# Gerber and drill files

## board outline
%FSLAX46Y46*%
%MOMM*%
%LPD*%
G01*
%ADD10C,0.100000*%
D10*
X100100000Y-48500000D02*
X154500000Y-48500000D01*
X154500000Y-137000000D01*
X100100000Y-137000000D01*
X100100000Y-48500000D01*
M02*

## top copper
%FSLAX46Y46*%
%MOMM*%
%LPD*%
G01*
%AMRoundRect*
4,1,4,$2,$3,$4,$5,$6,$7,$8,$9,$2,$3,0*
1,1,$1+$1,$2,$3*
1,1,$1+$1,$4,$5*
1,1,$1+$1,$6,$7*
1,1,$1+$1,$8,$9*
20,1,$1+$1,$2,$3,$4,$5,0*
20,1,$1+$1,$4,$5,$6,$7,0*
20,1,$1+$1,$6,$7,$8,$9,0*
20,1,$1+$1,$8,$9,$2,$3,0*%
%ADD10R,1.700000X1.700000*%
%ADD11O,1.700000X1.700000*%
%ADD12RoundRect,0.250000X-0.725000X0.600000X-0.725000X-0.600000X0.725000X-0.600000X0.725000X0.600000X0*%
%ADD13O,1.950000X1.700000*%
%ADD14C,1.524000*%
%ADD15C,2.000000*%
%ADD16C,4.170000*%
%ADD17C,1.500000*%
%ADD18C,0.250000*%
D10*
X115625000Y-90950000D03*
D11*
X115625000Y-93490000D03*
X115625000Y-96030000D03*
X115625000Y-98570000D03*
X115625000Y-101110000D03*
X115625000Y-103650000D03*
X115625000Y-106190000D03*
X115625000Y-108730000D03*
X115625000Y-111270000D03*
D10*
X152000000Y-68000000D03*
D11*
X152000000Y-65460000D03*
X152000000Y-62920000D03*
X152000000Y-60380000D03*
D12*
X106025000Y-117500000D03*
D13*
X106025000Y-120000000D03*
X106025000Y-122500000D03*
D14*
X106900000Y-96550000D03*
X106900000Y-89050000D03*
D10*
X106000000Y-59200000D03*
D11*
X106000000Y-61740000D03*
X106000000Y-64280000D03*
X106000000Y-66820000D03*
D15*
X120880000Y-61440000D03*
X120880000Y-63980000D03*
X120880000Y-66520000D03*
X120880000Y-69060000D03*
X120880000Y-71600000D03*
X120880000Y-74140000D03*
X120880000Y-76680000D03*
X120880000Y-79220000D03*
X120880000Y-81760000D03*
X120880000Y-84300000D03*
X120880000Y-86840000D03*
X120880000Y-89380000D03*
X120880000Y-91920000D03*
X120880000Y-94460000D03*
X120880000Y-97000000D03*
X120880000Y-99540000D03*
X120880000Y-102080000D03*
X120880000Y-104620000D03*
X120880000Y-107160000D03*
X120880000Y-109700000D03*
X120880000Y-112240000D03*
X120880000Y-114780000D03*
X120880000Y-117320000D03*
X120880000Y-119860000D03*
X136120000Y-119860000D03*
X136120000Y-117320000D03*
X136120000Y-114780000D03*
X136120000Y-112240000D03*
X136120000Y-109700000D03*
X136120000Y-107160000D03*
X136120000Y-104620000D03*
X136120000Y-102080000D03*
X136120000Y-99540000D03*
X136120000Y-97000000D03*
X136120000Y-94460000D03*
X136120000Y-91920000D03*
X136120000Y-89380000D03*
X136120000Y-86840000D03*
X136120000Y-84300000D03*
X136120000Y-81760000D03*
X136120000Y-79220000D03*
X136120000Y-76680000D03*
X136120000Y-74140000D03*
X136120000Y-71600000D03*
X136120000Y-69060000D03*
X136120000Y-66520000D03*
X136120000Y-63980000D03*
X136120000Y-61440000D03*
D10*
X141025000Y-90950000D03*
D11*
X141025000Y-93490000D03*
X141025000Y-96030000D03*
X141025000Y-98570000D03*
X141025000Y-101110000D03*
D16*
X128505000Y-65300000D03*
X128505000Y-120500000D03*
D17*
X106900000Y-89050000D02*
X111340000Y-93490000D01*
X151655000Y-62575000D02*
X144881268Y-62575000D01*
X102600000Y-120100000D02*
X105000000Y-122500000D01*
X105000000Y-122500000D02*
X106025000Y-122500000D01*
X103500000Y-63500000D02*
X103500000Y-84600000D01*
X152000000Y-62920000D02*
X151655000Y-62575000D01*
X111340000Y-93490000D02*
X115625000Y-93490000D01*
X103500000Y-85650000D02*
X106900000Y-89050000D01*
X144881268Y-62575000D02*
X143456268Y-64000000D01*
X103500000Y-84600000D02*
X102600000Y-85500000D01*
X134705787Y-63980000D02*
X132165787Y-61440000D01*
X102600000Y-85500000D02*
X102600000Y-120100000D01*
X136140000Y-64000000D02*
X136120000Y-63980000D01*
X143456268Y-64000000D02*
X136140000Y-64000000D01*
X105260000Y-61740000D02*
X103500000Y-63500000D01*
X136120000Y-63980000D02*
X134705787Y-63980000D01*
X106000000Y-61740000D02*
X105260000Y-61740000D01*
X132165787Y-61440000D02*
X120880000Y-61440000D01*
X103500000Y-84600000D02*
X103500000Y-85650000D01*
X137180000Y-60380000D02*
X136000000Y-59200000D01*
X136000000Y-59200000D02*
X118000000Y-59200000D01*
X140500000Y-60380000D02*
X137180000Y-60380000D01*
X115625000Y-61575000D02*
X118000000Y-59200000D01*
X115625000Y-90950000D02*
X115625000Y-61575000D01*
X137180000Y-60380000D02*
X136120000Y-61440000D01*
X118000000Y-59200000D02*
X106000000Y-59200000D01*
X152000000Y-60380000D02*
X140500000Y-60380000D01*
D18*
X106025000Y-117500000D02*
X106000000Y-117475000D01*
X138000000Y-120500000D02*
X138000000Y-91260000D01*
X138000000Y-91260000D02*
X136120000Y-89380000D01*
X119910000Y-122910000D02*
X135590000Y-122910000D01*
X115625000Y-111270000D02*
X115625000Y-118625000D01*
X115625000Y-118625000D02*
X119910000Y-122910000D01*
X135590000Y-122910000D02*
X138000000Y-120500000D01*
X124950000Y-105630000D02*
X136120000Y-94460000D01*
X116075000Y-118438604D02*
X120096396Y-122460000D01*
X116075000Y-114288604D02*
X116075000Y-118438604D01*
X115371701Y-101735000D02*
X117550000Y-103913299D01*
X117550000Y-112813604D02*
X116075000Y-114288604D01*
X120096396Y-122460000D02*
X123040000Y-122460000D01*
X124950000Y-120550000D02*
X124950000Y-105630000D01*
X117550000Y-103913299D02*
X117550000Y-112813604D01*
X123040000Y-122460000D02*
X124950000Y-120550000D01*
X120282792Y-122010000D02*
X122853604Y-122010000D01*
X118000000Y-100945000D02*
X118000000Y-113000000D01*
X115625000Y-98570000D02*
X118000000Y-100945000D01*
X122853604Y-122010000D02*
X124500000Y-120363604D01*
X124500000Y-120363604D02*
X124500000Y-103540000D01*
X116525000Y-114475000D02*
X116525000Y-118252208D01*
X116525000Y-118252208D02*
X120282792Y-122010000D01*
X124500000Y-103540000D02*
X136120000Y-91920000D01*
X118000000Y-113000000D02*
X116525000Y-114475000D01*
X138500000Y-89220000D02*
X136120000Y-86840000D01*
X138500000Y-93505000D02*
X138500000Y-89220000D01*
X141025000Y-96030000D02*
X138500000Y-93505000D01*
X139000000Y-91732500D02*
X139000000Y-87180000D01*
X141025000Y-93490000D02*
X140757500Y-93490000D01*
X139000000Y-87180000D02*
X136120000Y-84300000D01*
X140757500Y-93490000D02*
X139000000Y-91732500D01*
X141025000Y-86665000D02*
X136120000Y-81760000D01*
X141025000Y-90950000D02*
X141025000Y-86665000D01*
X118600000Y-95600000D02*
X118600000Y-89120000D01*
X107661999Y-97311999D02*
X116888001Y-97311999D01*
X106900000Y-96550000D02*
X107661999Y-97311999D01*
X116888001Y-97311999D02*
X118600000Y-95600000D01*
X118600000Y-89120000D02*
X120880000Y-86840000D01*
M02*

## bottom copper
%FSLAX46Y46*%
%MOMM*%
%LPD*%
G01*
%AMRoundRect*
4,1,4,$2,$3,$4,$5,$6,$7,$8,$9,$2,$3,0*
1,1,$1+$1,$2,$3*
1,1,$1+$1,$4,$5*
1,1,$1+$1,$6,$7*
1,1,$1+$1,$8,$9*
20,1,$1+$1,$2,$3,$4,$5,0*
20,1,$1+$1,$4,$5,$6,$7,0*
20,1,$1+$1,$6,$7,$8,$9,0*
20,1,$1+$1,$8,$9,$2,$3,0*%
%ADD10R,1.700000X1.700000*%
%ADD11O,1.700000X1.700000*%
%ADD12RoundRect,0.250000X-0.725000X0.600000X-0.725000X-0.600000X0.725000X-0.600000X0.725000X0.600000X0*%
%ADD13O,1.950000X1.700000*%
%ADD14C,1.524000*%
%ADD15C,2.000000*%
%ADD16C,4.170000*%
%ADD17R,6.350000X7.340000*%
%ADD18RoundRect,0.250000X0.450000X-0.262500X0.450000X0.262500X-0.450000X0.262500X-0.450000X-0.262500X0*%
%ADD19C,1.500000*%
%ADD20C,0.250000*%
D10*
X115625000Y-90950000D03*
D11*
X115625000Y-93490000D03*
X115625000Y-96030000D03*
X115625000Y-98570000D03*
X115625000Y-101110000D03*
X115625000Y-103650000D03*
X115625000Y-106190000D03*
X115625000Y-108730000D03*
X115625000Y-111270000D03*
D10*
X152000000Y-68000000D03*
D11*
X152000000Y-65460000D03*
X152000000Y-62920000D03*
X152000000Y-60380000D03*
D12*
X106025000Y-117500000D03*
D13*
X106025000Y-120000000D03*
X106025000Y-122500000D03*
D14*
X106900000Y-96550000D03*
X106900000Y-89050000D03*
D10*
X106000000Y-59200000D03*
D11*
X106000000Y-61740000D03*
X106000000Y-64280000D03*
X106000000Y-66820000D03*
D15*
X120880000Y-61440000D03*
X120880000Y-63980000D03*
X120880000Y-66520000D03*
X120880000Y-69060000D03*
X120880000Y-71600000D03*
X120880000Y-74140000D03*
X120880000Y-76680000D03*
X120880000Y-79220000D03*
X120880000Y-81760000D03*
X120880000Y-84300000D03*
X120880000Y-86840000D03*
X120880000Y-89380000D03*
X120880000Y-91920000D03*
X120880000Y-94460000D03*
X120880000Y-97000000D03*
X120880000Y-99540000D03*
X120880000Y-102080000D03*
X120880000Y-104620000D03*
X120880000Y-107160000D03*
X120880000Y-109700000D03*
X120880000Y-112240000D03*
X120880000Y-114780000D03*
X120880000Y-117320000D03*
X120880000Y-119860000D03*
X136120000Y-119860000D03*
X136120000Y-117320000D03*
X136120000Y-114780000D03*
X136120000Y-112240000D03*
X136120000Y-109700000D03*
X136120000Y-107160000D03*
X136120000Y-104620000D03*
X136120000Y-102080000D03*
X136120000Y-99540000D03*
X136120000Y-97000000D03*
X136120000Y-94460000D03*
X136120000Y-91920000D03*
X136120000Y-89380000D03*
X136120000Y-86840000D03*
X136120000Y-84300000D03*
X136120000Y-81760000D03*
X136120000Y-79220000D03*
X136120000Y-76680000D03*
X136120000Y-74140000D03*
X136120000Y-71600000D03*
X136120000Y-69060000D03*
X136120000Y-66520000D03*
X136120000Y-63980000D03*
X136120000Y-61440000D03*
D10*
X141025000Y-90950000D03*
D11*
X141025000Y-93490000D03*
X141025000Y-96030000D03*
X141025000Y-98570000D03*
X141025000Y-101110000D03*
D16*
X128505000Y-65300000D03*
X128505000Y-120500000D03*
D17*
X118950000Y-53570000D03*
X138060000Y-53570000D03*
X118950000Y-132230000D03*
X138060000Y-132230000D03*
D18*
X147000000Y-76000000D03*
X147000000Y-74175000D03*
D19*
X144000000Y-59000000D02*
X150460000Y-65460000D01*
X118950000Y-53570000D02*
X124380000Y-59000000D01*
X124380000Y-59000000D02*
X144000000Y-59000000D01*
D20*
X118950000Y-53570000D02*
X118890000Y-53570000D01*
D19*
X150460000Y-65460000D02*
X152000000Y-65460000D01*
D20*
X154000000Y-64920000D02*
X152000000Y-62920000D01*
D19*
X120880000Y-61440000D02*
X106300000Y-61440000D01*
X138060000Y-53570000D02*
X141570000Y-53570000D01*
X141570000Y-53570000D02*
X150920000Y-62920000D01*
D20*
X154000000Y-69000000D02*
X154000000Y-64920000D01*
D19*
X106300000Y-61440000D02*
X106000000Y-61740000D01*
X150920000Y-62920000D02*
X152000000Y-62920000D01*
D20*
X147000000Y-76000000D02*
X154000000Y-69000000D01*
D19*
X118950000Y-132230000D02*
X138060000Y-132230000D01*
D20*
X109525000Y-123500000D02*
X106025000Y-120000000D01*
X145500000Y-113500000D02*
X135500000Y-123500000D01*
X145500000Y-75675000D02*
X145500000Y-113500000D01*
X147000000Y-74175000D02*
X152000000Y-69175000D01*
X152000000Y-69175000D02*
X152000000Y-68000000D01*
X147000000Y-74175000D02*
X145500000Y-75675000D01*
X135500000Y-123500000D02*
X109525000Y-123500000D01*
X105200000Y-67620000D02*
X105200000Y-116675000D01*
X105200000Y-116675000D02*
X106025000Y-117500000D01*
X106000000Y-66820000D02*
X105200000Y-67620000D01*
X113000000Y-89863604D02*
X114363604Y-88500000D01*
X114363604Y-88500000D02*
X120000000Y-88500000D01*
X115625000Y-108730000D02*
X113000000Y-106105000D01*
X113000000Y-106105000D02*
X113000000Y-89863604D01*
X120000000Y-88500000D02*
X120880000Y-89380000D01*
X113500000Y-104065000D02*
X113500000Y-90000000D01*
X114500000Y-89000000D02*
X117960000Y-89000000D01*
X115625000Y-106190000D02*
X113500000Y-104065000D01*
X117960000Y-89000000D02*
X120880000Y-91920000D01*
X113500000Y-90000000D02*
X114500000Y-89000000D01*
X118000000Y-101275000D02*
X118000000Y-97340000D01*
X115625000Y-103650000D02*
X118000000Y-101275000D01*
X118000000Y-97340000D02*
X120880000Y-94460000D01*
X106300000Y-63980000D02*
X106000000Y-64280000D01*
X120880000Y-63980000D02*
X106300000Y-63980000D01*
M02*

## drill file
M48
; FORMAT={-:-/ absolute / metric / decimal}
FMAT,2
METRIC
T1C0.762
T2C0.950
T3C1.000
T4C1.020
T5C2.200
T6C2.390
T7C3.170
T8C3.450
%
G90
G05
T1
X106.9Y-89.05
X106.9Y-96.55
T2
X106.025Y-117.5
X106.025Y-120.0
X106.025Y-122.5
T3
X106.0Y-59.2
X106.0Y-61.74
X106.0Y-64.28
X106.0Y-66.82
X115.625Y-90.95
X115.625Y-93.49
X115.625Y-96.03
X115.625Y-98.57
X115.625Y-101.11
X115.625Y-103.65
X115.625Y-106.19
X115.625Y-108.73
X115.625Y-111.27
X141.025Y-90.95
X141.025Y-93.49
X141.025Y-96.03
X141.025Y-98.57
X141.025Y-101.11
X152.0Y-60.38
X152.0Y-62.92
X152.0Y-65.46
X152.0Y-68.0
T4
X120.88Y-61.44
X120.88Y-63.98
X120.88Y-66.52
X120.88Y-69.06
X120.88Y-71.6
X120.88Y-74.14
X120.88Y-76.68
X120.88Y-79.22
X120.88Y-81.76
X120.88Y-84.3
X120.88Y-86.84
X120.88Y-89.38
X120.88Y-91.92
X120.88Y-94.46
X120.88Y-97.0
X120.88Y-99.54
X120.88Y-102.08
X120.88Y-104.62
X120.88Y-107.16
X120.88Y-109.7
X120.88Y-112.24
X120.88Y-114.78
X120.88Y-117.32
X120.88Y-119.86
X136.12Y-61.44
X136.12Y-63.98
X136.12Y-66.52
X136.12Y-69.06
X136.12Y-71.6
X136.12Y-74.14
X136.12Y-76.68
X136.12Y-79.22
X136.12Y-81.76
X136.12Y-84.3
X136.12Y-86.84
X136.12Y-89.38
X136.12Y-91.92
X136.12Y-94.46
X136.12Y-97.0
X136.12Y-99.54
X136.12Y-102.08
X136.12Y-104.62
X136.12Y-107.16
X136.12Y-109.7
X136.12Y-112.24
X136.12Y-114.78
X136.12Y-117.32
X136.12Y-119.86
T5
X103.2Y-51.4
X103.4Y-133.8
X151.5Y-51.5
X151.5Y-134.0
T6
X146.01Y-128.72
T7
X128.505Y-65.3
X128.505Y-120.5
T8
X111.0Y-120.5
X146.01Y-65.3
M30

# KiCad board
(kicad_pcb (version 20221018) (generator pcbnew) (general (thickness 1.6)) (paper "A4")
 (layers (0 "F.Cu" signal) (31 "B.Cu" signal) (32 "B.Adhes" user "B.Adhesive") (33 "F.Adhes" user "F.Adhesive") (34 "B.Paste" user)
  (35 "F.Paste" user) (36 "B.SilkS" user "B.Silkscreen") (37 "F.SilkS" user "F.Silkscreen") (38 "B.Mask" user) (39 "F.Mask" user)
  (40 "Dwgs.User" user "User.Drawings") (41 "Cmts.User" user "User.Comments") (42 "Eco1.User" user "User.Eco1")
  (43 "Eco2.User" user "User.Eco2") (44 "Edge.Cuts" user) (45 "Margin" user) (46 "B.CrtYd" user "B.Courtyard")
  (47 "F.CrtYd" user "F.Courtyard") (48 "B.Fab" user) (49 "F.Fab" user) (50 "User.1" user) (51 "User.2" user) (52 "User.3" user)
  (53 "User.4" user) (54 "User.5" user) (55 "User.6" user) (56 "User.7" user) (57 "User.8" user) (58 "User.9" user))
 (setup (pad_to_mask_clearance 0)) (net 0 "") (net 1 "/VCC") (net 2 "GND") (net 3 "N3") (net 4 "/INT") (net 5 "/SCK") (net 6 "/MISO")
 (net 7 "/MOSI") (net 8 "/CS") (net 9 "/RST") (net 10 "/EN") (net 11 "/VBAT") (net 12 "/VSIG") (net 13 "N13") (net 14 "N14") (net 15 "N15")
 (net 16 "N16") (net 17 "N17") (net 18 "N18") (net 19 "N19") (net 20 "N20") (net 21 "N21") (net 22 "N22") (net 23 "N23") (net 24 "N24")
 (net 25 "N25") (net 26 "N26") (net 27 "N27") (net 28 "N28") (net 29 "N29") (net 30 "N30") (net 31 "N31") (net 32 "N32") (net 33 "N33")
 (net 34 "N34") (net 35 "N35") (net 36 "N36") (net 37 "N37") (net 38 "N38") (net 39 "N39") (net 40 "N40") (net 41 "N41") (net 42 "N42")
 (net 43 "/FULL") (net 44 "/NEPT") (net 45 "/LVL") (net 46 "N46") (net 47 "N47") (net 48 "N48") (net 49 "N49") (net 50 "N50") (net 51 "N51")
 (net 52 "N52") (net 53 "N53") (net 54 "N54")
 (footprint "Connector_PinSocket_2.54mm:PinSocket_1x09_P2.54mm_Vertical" (layer "F.Cu") (at 115.625 90.95)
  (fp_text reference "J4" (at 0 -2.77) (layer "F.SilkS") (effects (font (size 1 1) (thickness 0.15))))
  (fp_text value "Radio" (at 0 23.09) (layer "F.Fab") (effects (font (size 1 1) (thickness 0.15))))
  (pad "1" thru_hole rect (at 0 0) (size 1.7 1.7) (drill 1) (layers "*.Cu" "*.Mask") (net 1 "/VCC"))
  (pad "2" thru_hole oval (at 0 2.54) (size 1.7 1.7) (drill 1) (layers "*.Cu" "*.Mask") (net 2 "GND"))
  (pad "3" thru_hole oval (at 0 5.08) (size 1.7 1.7) (drill 1) (layers "*.Cu" "*.Mask") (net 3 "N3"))
  (pad "4" thru_hole oval (at 0 7.62) (size 1.7 1.7) (drill 1) (layers "*.Cu" "*.Mask") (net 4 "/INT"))
  (pad "5" thru_hole oval (at 0 10.16) (size 1.7 1.7) (drill 1) (layers "*.Cu" "*.Mask") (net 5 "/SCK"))
  (pad "6" thru_hole oval (at 0 12.7) (size 1.7 1.7) (drill 1) (layers "*.Cu" "*.Mask") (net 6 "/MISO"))
  (pad "7" thru_hole oval (at 0 15.24) (size 1.7 1.7) (drill 1) (layers "*.Cu" "*.Mask") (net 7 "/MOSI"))
  (pad "8" thru_hole oval (at 0 17.78) (size 1.7 1.7) (drill 1) (layers "*.Cu" "*.Mask") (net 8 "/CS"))
  (pad "9" thru_hole oval (at 0 20.32) (size 1.7 1.7) (drill 1) (layers "*.Cu" "*.Mask") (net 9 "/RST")))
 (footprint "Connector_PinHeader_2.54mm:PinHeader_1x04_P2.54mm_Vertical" (layer "F.Cu") (at 152 68 180)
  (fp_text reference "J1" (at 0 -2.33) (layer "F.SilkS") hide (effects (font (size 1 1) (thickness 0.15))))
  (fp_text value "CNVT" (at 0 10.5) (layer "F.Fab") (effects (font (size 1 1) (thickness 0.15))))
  (pad "1" thru_hole rect (at 0 0 180) (size 1.7 1.7) (drill 1) (layers "*.Cu" "*.Mask") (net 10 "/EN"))
  (pad "2" thru_hole oval (at 0 2.54 180) (size 1.7 1.7) (drill 1) (layers "*.Cu" "*.Mask") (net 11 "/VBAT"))
  (pad "3" thru_hole oval (at 0 5.08 180) (size 1.7 1.7) (drill 1) (layers "*.Cu" "*.Mask") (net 2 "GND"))
  (pad "4" thru_hole oval (at 0 7.62 180) (size 1.7 1.7) (drill 1) (layers "*.Cu" "*.Mask") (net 1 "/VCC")))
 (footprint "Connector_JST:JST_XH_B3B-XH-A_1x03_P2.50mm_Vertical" (layer "F.Cu") (at 106.025 117.5 -90)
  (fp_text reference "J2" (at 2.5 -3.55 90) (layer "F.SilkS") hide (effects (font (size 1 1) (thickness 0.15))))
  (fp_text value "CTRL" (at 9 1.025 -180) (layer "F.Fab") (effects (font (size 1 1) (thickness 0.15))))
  (pad "1" thru_hole roundrect (at 0 0 270) (size 1.7 1.95) (drill 0.95) (layers "*.Cu" "*.Mask") (roundrect_rratio 0.1470588235)
   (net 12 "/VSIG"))
  (pad "2" thru_hole oval (at 2.5 0 270) (size 1.7 1.95) (drill 0.95) (layers "*.Cu" "*.Mask") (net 10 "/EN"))
  (pad "3" thru_hole oval (at 5 0 270) (size 1.7 1.95) (drill 0.95) (layers "*.Cu" "*.Mask") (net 2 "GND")))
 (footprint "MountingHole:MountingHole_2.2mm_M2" (layer "F.Cu") (at 151.5 134)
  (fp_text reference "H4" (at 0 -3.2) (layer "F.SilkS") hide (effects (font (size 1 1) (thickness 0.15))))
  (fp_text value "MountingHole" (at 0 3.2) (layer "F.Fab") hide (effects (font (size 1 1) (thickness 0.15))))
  (pad "" np_thru_hole circle (at 0 0) (size 2.2 2.2) (drill 2.2) (layers "*.Cu" "*.Mask")))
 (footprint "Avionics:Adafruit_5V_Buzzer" (layer "F.Cu") (at 111.4 92.8 90)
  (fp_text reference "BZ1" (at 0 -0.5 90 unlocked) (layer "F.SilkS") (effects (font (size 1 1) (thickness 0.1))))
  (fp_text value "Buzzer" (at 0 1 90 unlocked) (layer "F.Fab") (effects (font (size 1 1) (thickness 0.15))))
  (pad "1" thru_hole circle (at -3.75 -4.5 90) (size 1.524 1.524) (drill 0.762) (layers "*.Cu" "*.Mask") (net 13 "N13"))
  (pad "2" thru_hole circle (at 3.75 -4.5 90) (size 1.524 1.524) (drill 0.762) (layers "*.Cu" "*.Mask") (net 2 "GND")))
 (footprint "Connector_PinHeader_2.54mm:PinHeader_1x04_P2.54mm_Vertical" (layer "F.Cu") (at 106 59.2)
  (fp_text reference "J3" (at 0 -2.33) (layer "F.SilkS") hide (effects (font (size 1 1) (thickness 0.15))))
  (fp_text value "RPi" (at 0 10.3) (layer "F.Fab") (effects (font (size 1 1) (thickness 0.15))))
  (pad "1" thru_hole rect (at 0 0) (size 1.7 1.7) (drill 1) (layers "*.Cu" "*.Mask") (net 1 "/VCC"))
  (pad "2" thru_hole oval (at 0 2.54) (size 1.7 1.7) (drill 1) (layers "*.Cu" "*.Mask") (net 2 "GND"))
  (pad "3" thru_hole oval (at 0 5.08) (size 1.7 1.7) (drill 1) (layers "*.Cu" "*.Mask") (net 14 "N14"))
  (pad "4" thru_hole oval (at 0 7.62) (size 1.7 1.7) (drill 1) (layers "*.Cu" "*.Mask") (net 12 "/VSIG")))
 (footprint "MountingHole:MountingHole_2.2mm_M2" (layer "F.Cu") (at 151.5 51.5)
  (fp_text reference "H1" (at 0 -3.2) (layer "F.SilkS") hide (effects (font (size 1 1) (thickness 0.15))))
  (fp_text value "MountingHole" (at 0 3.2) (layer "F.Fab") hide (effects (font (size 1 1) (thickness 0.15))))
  (pad "" np_thru_hole circle (at 0 0) (size 2.2 2.2) (drill 2.2) (layers "*.Cu" "*.Mask")))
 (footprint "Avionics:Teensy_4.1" (layer "F.Cu") (at 128.5 90.65)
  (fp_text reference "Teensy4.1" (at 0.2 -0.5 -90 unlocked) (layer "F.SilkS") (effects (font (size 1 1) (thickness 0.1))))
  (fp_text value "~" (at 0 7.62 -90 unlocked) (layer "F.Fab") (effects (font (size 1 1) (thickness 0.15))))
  (pad "0" thru_hole circle (at -7.62 -29.21) (size 2 2) (drill 1.02) (layers "*.Cu" "*.Mask") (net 2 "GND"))
  (pad "1" thru_hole circle (at -7.62 -26.67) (size 2 2) (drill 1.02) (layers "*.Cu" "*.Mask") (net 14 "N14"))
  (pad "2" thru_hole circle (at -7.62 -24.13) (size 2 2) (drill 1.02) (layers "*.Cu" "*.Mask") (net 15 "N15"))
  (pad "3" thru_hole circle (at -7.62 -21.59) (size 2 2) (drill 1.02) (layers "*.Cu" "*.Mask") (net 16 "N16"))
  (pad "4" thru_hole circle (at -7.62 -19.05) (size 2 2) (drill 1.02) (layers "*.Cu" "*.Mask") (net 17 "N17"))
  (pad "5" thru_hole circle (at -7.62 -16.51) (size 2 2) (drill 1.02) (layers "*.Cu" "*.Mask") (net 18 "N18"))
  (pad "6" thru_hole circle (at -7.62 -13.97) (size 2 2) (drill 1.02) (layers "*.Cu" "*.Mask") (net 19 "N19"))
  (pad "7" thru_hole circle (at -7.62 -11.43) (size 2 2) (drill 1.02) (layers "*.Cu" "*.Mask") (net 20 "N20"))
  (pad "8" thru_hole circle (at -7.62 -8.89) (size 2 2) (drill 1.02) (layers "*.Cu" "*.Mask") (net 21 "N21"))
  (pad "9" thru_hole circle (at -7.62 -6.35) (size 2 2) (drill 1.02) (layers "*.Cu" "*.Mask") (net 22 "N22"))
  (pad "10" thru_hole circle (at -7.62 -3.81) (size 2 2) (drill 1.02) (layers "*.Cu" "*.Mask") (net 13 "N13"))
  (pad "11" thru_hole circle (at -7.62 -1.27) (size 2 2) (drill 1.02) (layers "*.Cu" "*.Mask") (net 8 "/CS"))
  (pad "12" thru_hole circle (at -7.62 1.27) (size 2 2) (drill 1.02) (layers "*.Cu" "*.Mask") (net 7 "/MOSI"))
  (pad "13" thru_hole circle (at -7.62 3.81) (size 2 2) (drill 1.02) (layers "*.Cu" "*.Mask") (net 6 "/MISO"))
  (pad "14" thru_hole circle (at -7.62 6.35) (size 2 2) (drill 1.02) (layers "*.Cu" "*.Mask") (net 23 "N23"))
  (pad "15" thru_hole circle (at -7.62 8.89) (size 2 2) (drill 1.02) (layers "*.Cu" "*.Mask") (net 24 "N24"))
  (pad "16" thru_hole circle (at -7.62 11.43) (size 2 2) (drill 1.02) (layers "*.Cu" "*.Mask") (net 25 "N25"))
  (pad "17" thru_hole circle (at -7.62 13.97) (size 2 2) (drill 1.02) (layers "*.Cu" "*.Mask") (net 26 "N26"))
  (pad "18" thru_hole circle (at -7.62 16.51) (size 2 2) (drill 1.02) (layers "*.Cu" "*.Mask") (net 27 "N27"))
  (pad "19" thru_hole circle (at -7.62 19.05) (size 2 2) (drill 1.02) (layers "*.Cu" "*.Mask") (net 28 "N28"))
  (pad "20" thru_hole circle (at -7.62 21.59) (size 2 2) (drill 1.02) (layers "*.Cu" "*.Mask") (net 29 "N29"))
  (pad "21" thru_hole circle (at -7.62 24.13) (size 2 2) (drill 1.02) (layers "*.Cu" "*.Mask") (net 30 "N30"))
  (pad "22" thru_hole circle (at -7.62 26.67) (size 2 2) (drill 1.02) (layers "*.Cu" "*.Mask") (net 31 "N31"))
  (pad "23" thru_hole circle (at -7.62 29.21) (size 2 2) (drill 1.02) (layers "*.Cu" "*.Mask") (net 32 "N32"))
  (pad "24" thru_hole circle (at 7.62 29.21) (size 2 2) (drill 1.02) (layers "*.Cu" "*.Mask") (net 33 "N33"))
  (pad "25" thru_hole circle (at 7.62 26.67) (size 2 2) (drill 1.02) (layers "*.Cu" "*.Mask") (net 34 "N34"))
  (pad "26" thru_hole circle (at 7.62 24.13) (size 2 2) (drill 1.02) (layers "*.Cu" "*.Mask") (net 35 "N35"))
  (pad "27" thru_hole circle (at 7.62 21.59) (size 2 2) (drill 1.02) (layers "*.Cu" "*.Mask") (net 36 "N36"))
  (pad "28" thru_hole circle (at 7.62 19.05) (size 2 2) (drill 1.02) (layers "*.Cu" "*.Mask") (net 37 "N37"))
  (pad "29" thru_hole circle (at 7.62 16.51) (size 2 2) (drill 1.02) (layers "*.Cu" "*.Mask") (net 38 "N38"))
  (pad "30" thru_hole circle (at 7.62 13.97) (size 2 2) (drill 1.02) (layers "*.Cu" "*.Mask") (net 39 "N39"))
  (pad "31" thru_hole circle (at 7.62 11.43) (size 2 2) (drill 1.02) (layers "*.Cu" "*.Mask") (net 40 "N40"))
  (pad "32" thru_hole circle (at 7.62 8.89) (size 2 2) (drill 1.02) (layers "*.Cu" "*.Mask") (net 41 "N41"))
  (pad "33" thru_hole circle (at 7.62 6.35) (size 2 2) (drill 1.02) (layers "*.Cu" "*.Mask") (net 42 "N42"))
  (pad "34" thru_hole circle (at 7.62 3.81) (size 2 2) (drill 1.02) (layers "*.Cu" "*.Mask") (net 5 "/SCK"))
  (pad "35" thru_hole circle (at 7.62 1.27) (size 2 2) (drill 1.02) (layers "*.Cu" "*.Mask") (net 4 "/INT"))
  (pad "36" thru_hole circle (at 7.62 -1.27) (size 2 2) (drill 1.02) (layers "*.Cu" "*.Mask") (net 9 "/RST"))
  (pad "37" thru_hole circle (at 7.62 -3.81) (size 2 2) (drill 1.02) (layers "*.Cu" "*.Mask") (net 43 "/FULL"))
  (pad "38" thru_hole circle (at 7.62 -6.35) (size 2 2) (drill 1.02) (layers "*.Cu" "*.Mask") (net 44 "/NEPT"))
  (pad "39" thru_hole circle (at 7.62 -8.89) (size 2 2) (drill 1.02) (layers "*.Cu" "*.Mask") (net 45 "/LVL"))
  (pad "40" thru_hole circle (at 7.62 -11.43) (size 2 2) (drill 1.02) (layers "*.Cu" "*.Mask") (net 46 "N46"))
  (pad "41" thru_hole circle (at 7.62 -13.97) (size 2 2) (drill 1.02) (layers "*.Cu" "*.Mask") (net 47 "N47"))
  (pad "42" thru_hole circle (at 7.62 -16.51) (size 2 2) (drill 1.02) (layers "*.Cu" "*.Mask") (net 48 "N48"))
  (pad "43" thru_hole circle (at 7.62 -19.05) (size 2 2) (drill 1.02) (layers "*.Cu" "*.Mask") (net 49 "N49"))
  (pad "44" thru_hole circle (at 7.62 -21.59) (size 2 2) (drill 1.02) (layers "*.Cu" "*.Mask") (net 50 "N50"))
  (pad "45" thru_hole circle (at 7.62 -24.13) (size 2 2) (drill 1.02) (layers "*.Cu" "*.Mask") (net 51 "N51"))
  (pad "46" thru_hole circle (at 7.62 -26.67) (size 2 2) (drill 1.02) (layers "*.Cu" "*.Mask") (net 2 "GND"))
  (pad "47" thru_hole circle (at 7.62 -29.21) (size 2 2) (drill 1.02) (layers "*.Cu" "*.Mask") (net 1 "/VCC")))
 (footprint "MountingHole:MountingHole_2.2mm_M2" (layer "F.Cu") (at 103.2 51.4)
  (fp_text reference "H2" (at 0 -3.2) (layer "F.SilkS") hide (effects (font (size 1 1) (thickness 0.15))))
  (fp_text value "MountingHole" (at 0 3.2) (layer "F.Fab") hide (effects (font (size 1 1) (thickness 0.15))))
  (pad "" np_thru_hole circle (at 0 0) (size 2.2 2.2) (drill 2.2) (layers "*.Cu" "*.Mask")))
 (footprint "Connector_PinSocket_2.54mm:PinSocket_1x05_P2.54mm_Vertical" (layer "F.Cu") (at 141.025 90.95)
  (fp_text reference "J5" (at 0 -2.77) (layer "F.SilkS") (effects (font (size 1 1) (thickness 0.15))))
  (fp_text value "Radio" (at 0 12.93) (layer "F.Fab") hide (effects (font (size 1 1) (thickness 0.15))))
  (pad "1" thru_hole rect (at 0 0) (size 1.7 1.7) (drill 1) (layers "*.Cu" "*.Mask") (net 45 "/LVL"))
  (pad "2" thru_hole oval (at 0 2.54) (size 1.7 1.7) (drill 1) (layers "*.Cu" "*.Mask") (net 44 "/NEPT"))
  (pad "3" thru_hole oval (at 0 5.08) (size 1.7 1.7) (drill 1) (layers "*.Cu" "*.Mask") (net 43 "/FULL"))
  (pad "4" thru_hole oval (at 0 7.62) (size 1.7 1.7) (drill 1) (layers "*.Cu" "*.Mask") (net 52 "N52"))
  (pad "5" thru_hole oval (at 0 10.16) (size 1.7 1.7) (drill 1) (layers "*.Cu" "*.Mask") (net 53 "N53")))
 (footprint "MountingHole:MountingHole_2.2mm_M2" (layer "F.Cu") (at 103.4 133.8)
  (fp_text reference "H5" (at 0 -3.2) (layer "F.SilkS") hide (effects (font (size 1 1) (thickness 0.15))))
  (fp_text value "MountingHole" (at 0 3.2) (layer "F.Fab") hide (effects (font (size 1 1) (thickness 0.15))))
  (pad "" np_thru_hole circle (at 0 0) (size 2.2 2.2) (drill 2.2) (layers "*.Cu" "*.Mask")))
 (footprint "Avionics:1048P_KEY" (layer "B.Cu") (at 128.505 92.9 -90)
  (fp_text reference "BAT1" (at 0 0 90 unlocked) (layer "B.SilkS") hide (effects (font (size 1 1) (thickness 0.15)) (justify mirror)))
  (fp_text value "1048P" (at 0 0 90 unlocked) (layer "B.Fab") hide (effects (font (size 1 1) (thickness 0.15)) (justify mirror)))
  (pad "" np_thru_hole circle (at -27.6 -17.505 270) (size 3.45 3.45) (drill 3.45) (layers "F&B.Cu" "*.Mask"))
  (pad "" np_thru_hole circle (at -27.6 0 270) (size 4.17 4.17) (drill 3.17) (layers "F&B.Cu" "*.Mask"))
  (pad "" np_thru_hole circle (at 27.6 0 270) (size 4.17 4.17) (drill 3.17) (layers "F&B.Cu" "*.Mask"))
  (pad "" np_thru_hole circle (at 27.6 17.505 270) (size 3.45 3.45) (drill 3.45) (layers "F&B.Cu" "*.Mask"))
  (pad "" np_thru_hole circle (at 35.82 -17.505 270) (size 2.39 2.39) (drill 2.39) (layers "F&B.Cu" "*.Mask"))
  (pad "1" smd rect (at -39.33 9.555 270) (size 7.34 6.35) (layers "B.Cu" "B.Paste" "B.Mask") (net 11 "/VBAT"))
  (pad "2" smd rect (at -39.33 -9.555 270) (size 7.34 6.35) (layers "B.Cu" "B.Paste" "B.Mask") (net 2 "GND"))
  (pad "3" smd rect (at 39.33 9.555 270) (size 7.34 6.35) (layers "B.Cu" "B.Paste" "B.Mask") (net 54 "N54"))
  (pad "4" smd rect (at 39.33 -9.555 270) (size 7.34 6.35) (layers "B.Cu" "B.Paste" "B.Mask") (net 54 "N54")))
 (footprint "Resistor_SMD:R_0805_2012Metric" (layer "B.Cu") (at 147 75.0875 90)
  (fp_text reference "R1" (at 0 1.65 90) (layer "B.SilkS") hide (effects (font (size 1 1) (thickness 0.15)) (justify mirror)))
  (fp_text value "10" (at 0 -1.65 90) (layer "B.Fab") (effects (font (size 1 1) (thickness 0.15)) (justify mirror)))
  (pad "1" smd roundrect (at -0.9125 0 90) (size 1.025 1.4) (layers "B.Cu" "B.Paste" "B.Mask") (roundrect_rratio 0.243902439) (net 2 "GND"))
  (pad "2" smd roundrect (at 0.9125 0 90) (size 1.025 1.4) (layers "B.Cu" "B.Paste" "B.Mask") (roundrect_rratio 0.243902439) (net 10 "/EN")))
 (gr_rect (start 100.1 48.5) (end 154.5 137) (stroke (width 0.1) (type default)) (fill none) (layer "Edge.Cuts"))
 (segment (start 144 59) (end 150.46 65.46) (width 1.5) (layer "B.Cu") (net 11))
 (segment (start 118.95 53.57) (end 124.38 59) (width 1.5) (layer "B.Cu") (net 11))
 (segment (start 124.38 59) (end 144 59) (width 1.5) (layer "B.Cu") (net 11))
 (segment (start 118.95 53.57) (end 118.89 53.57) (width 0.25) (layer "B.Cu") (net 11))
 (segment (start 150.46 65.46) (end 152 65.46) (width 1.5) (layer "B.Cu") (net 11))
 (segment (start 106.9 89.05) (end 111.34 93.49) (width 1.5) (layer "F.Cu") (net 2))
 (segment (start 151.655 62.575) (end 144.881268 62.575) (width 1.5) (layer "F.Cu") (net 2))
 (segment (start 102.6 120.1) (end 105 122.5) (width 1.5) (layer "F.Cu") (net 2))
 (segment (start 105 122.5) (end 106.025 122.5) (width 1.5) (layer "F.Cu") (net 2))
 (segment (start 103.5 63.5) (end 103.5 84.6) (width 1.5) (layer "F.Cu") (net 2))
 (segment (start 152 62.92) (end 151.655 62.575) (width 1.5) (layer "F.Cu") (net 2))
 (segment (start 111.34 93.49) (end 115.625 93.49) (width 1.5) (layer "F.Cu") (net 2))
 (segment (start 103.5 85.65) (end 106.9 89.05) (width 1.5) (layer "F.Cu") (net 2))
 (segment (start 144.881268 62.575) (end 143.456268 64) (width 1.5) (layer "F.Cu") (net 2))
 (segment (start 103.5 84.6) (end 102.6 85.5) (width 1.5) (layer "F.Cu") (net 2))
 (segment (start 134.705787 63.98) (end 132.165787 61.44) (width 1.5) (layer "F.Cu") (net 2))
 (segment (start 102.6 85.5) (end 102.6 120.1) (width 1.5) (layer "F.Cu") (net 2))
 (segment (start 136.14 64) (end 136.12 63.98) (width 1.5) (layer "F.Cu") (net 2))
 (segment (start 143.456268 64) (end 136.14 64) (width 1.5) (layer "F.Cu") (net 2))
 (segment (start 105.26 61.74) (end 103.5 63.5) (width 1.5) (layer "F.Cu") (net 2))
 (segment (start 136.12 63.98) (end 134.705787 63.98) (width 1.5) (layer "F.Cu") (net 2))
 (segment (start 106 61.74) (end 105.26 61.74) (width 1.5) (layer "F.Cu") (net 2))
 (segment (start 132.165787 61.44) (end 120.88 61.44) (width 1.5) (layer "F.Cu") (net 2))
 (segment (start 103.5 84.6) (end 103.5 85.65) (width 1.5) (layer "F.Cu") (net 2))
 (segment (start 154 64.92) (end 152 62.92) (width 0.25) (layer "B.Cu") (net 2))
 (segment (start 120.88 61.44) (end 106.3 61.44) (width 1.5) (layer "B.Cu") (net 2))
 (segment (start 138.06 53.57) (end 141.57 53.57) (width 1.5) (layer "B.Cu") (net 2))
 (segment (start 141.57 53.57) (end 150.92 62.92) (width 1.5) (layer "B.Cu") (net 2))
 (segment (start 154 69) (end 154 64.92) (width 0.25) (layer "B.Cu") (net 2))
 (segment (start 106.3 61.44) (end 106 61.74) (width 1.5) (layer "B.Cu") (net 2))
 (segment (start 150.92 62.92) (end 152 62.92) (width 1.5) (layer "B.Cu") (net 2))
 (segment (start 147 76) (end 154 69) (width 0.25) (layer "B.Cu") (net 2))
 (segment (start 118.95 132.23) (end 138.06 132.23) (width 1.5) (layer "B.Cu") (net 54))
 (segment (start 109.525 123.5) (end 106.025 120) (width 0.25) (layer "B.Cu") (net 10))
 (segment (start 145.5 113.5) (end 135.5 123.5) (width 0.25) (layer "B.Cu") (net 10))
 (segment (start 145.5 75.675) (end 145.5 113.5) (width 0.25) (layer "B.Cu") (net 10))
 (segment (start 147 74.175) (end 152 69.175) (width 0.25) (layer "B.Cu") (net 10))
 (segment (start 152 69.175) (end 152 68) (width 0.25) (layer "B.Cu") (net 10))
 (segment (start 147 74.175) (end 145.5 75.675) (width 0.25) (layer "B.Cu") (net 10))
 (segment (start 135.5 123.5) (end 109.525 123.5) (width 0.25) (layer "B.Cu") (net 10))
 (segment (start 137.18 60.38) (end 136 59.2) (width 1.5) (layer "F.Cu") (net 1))
 (segment (start 136 59.2) (end 118 59.2) (width 1.5) (layer "F.Cu") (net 1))
 (segment (start 140.5 60.38) (end 137.18 60.38) (width 1.5) (layer "F.Cu") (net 1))
 (segment (start 115.625 61.575) (end 118 59.2) (width 1.5) (layer "F.Cu") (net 1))
 (segment (start 115.625 90.95) (end 115.625 61.575) (width 1.5) (layer "F.Cu") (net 1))
 (segment (start 137.18 60.38) (end 136.12 61.44) (width 1.5) (layer "F.Cu") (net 1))
 (segment (start 118 59.2) (end 106 59.2) (width 1.5) (layer "F.Cu") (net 1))
 (segment (start 152 60.38) (end 140.5 60.38) (width 1.5) (layer "F.Cu") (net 1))
 (segment (start 106.025 117.5) (end 106 117.475) (width 0.25) (layer "F.Cu") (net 12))
 (segment (start 105.2 67.62) (end 105.2 116.675) (width 0.25) (layer "B.Cu") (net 12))
 (segment (start 105.2 116.675) (end 106.025 117.5) (width 0.25) (layer "B.Cu") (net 12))
 (segment (start 106 66.82) (end 105.2 67.62) (width 0.25) (layer "B.Cu") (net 12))
 (segment (start 138 120.5) (end 138 91.26) (width 0.25) (layer "F.Cu") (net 9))
 (segment (start 138 91.26) (end 136.12 89.38) (width 0.25) (layer "F.Cu") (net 9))
 (segment (start 119.91 122.91) (end 135.59 122.91) (width 0.25) (layer "F.Cu") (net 9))
 (segment (start 115.625 111.27) (end 115.625 118.625) (width 0.25) (layer "F.Cu") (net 9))
 (segment (start 115.625 118.625) (end 119.91 122.91) (width 0.25) (layer "F.Cu") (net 9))
 (segment (start 135.59 122.91) (end 138 120.5) (width 0.25) (layer "F.Cu") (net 9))
 (segment (start 113 89.863604) (end 114.363604 88.5) (width 0.25) (layer "B.Cu") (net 8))
 (segment (start 114.363604 88.5) (end 120 88.5) (width 0.25) (layer "B.Cu") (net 8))
 (segment (start 115.625 108.73) (end 113 106.105) (width 0.25) (layer "B.Cu") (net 8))
 (segment (start 113 106.105) (end 113 89.863604) (width 0.25) (layer "B.Cu") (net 8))
 (segment (start 120 88.5) (end 120.88 89.38) (width 0.25) (layer "B.Cu") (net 8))
 (segment (start 113.5 104.065) (end 113.5 90) (width 0.25) (layer "B.Cu") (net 7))
 (segment (start 114.5 89) (end 117.96 89) (width 0.25) (layer "B.Cu") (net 7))
 (segment (start 115.625 106.19) (end 113.5 104.065) (width 0.25) (layer "B.Cu") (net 7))
 (segment (start 117.96 89) (end 120.88 91.92) (width 0.25) (layer "B.Cu") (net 7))
 (segment (start 113.5 90) (end 114.5 89) (width 0.25) (layer "B.Cu") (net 7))
 (segment (start 118 101.275) (end 118 97.34) (width 0.25) (layer "B.Cu") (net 6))
 (segment (start 115.625 103.65) (end 118 101.275) (width 0.25) (layer "B.Cu") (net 6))
 (segment (start 118 97.34) (end 120.88 94.46) (width 0.25) (layer "B.Cu") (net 6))
 (segment (start 124.95 105.63) (end 136.12 94.46) (width 0.25) (layer "F.Cu") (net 5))
 (segment (start 116.075 118.438604) (end 120.096396 122.46) (width 0.25) (layer "F.Cu") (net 5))
 (segment (start 116.075 114.288604) (end 116.075 118.438604) (width 0.25) (layer "F.Cu") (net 5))
 (segment (start 115.371701 101.735) (end 117.55 103.913299) (width 0.25) (layer "F.Cu") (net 5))
 (segment (start 117.55 112.813604) (end 116.075 114.288604) (width 0.25) (layer "F.Cu") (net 5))
 (segment (start 120.096396 122.46) (end 123.04 122.46) (width 0.25) (layer "F.Cu") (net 5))
 (segment (start 124.95 120.55) (end 124.95 105.63) (width 0.25) (layer "F.Cu") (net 5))
 (segment (start 117.55 103.913299) (end 117.55 112.813604) (width 0.25) (layer "F.Cu") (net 5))
 (segment (start 123.04 122.46) (end 124.95 120.55) (width 0.25) (layer "F.Cu") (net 5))
 (segment (start 120.282792 122.01) (end 122.853604 122.01) (width 0.25) (layer "F.Cu") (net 4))
 (segment (start 118 100.945) (end 118 113) (width 0.25) (layer "F.Cu") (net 4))
 (segment (start 115.625 98.57) (end 118 100.945) (width 0.25) (layer "F.Cu") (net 4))
 (segment (start 122.853604 122.01) (end 124.5 120.363604) (width 0.25) (layer "F.Cu") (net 4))
 (segment (start 124.5 120.363604) (end 124.5 103.54) (width 0.25) (layer "F.Cu") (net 4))
 (segment (start 116.525 114.475) (end 116.525 118.252208) (width 0.25) (layer "F.Cu") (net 4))
 (segment (start 116.525 118.252208) (end 120.282792 122.01) (width 0.25) (layer "F.Cu") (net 4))
 (segment (start 124.5 103.54) (end 136.12 91.92) (width 0.25) (layer "F.Cu") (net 4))
 (segment (start 118 113) (end 116.525 114.475) (width 0.25) (layer "F.Cu") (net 4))
 (segment (start 138.5 89.22) (end 136.12 86.84) (width 0.25) (layer "F.Cu") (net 43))
 (segment (start 138.5 93.505) (end 138.5 89.22) (width 0.25) (layer "F.Cu") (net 43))
 (segment (start 141.025 96.03) (end 138.5 93.505) (width 0.25) (layer "F.Cu") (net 43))
 (segment (start 139 91.7325) (end 139 87.18) (width 0.25) (layer "F.Cu") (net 44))
 (segment (start 141.025 93.49) (end 140.7575 93.49) (width 0.25) (layer "F.Cu") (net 44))
 (segment (start 139 87.18) (end 136.12 84.3) (width 0.25) (layer "F.Cu") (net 44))
 (segment (start 140.7575 93.49) (end 139 91.7325) (width 0.25) (layer "F.Cu") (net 44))
 (segment (start 141.025 86.665) (end 136.12 81.76) (width 0.25) (layer "F.Cu") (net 45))
 (segment (start 141.025 90.95) (end 141.025 86.665) (width 0.25) (layer "F.Cu") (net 45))
 (segment (start 118.6 95.6) (end 118.6 89.12) (width 0.25) (layer "F.Cu") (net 13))
 (segment (start 107.661999 97.311999) (end 116.888001 97.311999) (width 0.25) (layer "F.Cu") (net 13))
 (segment (start 106.9 96.55) (end 107.661999 97.311999) (width 0.25) (layer "F.Cu") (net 13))
 (segment (start 116.888001 97.311999) (end 118.6 95.6) (width 0.25) (layer "F.Cu") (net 13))
 (segment (start 118.6 89.12) (end 120.88 86.84) (width 0.25) (layer "F.Cu") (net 13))
 (segment (start 106.3 63.98) (end 106 64.28) (width 0.25) (layer "B.Cu") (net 14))
 (segment (start 120.88 63.98) (end 106.3 63.98) (width 0.25) (layer "B.Cu") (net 14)))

